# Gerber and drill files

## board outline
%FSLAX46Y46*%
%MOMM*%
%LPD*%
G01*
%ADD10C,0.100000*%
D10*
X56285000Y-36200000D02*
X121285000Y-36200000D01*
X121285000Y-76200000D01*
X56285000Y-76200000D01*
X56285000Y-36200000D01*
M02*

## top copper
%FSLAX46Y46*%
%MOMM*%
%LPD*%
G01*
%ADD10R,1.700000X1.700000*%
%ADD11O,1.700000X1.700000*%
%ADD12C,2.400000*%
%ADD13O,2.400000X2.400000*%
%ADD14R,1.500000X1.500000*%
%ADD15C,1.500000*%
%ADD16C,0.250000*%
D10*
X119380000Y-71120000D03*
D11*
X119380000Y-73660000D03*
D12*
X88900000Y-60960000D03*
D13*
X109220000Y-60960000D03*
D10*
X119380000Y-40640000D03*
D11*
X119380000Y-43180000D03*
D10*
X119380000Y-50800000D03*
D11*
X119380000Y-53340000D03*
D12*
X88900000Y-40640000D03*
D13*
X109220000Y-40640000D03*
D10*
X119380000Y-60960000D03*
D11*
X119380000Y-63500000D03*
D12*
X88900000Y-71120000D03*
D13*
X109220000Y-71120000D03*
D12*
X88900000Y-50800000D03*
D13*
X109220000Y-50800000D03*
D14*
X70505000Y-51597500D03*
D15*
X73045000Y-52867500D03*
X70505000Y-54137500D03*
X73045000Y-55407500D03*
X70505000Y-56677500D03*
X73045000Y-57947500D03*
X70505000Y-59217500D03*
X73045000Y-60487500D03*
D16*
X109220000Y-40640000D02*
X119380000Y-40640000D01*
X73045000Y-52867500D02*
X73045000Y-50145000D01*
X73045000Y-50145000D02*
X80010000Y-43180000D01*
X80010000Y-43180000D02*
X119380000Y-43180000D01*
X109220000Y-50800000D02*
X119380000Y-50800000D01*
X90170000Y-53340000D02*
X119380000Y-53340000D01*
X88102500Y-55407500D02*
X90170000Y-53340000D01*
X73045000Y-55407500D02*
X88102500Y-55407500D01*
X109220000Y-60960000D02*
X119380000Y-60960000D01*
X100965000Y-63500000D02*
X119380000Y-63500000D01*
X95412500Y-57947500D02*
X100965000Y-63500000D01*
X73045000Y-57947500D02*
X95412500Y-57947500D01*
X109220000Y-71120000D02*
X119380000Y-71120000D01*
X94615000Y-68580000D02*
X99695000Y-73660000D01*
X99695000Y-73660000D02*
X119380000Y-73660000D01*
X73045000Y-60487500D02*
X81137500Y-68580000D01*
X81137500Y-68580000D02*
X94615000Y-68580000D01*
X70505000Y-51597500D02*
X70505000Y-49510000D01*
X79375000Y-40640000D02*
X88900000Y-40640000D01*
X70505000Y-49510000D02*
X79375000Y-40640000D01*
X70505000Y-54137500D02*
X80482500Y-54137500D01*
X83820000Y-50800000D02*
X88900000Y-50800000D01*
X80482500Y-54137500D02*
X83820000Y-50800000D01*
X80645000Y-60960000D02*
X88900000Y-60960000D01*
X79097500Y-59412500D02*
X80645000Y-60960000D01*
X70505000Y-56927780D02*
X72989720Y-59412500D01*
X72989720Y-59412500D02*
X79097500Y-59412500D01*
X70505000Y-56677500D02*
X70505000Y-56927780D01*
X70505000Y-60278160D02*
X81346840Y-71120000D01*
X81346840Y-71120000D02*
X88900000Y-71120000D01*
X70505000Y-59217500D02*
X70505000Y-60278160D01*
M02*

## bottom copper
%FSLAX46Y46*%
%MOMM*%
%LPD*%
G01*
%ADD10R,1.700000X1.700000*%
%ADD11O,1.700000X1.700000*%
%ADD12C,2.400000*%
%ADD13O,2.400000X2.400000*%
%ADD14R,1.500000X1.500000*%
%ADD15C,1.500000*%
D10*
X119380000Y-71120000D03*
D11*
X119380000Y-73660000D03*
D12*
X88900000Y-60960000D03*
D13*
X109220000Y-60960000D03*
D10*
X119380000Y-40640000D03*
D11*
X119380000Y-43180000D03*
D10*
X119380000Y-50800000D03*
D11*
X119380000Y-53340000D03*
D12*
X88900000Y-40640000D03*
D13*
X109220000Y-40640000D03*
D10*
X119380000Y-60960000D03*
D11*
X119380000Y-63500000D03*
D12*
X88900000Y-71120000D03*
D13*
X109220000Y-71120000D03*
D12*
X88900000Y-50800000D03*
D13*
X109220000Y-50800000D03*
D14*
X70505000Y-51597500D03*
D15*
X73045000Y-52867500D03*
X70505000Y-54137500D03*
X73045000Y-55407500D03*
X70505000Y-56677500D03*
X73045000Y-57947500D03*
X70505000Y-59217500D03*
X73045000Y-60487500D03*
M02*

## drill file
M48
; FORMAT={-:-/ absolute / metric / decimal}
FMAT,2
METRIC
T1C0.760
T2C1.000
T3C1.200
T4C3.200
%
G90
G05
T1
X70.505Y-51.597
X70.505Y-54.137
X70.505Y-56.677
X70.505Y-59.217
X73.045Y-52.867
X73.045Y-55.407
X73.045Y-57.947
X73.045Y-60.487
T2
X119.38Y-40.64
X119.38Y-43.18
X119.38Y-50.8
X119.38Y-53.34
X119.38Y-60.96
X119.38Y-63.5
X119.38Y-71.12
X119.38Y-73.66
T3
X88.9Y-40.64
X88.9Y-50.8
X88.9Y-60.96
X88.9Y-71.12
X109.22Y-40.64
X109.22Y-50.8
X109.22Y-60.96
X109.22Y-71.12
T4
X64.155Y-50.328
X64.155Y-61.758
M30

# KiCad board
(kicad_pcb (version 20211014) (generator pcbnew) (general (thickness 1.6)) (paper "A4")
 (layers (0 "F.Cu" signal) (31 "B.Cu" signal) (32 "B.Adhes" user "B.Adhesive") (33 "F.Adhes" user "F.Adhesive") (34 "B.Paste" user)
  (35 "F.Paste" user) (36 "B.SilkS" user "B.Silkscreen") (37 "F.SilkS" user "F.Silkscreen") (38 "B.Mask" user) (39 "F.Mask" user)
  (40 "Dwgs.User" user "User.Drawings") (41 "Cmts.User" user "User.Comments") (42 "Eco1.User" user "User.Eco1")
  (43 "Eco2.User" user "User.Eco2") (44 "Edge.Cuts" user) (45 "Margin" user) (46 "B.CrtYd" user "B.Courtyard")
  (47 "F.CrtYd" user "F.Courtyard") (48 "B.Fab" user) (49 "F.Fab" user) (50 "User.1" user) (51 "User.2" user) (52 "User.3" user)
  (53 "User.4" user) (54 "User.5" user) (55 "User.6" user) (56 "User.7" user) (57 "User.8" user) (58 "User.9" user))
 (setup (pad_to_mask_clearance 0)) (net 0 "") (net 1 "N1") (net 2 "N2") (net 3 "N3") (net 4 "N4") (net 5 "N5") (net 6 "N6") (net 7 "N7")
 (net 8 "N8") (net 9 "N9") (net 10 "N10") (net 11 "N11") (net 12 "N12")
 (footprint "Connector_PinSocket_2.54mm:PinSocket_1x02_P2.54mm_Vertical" (layer "F.Cu") (at 119.38 71.12)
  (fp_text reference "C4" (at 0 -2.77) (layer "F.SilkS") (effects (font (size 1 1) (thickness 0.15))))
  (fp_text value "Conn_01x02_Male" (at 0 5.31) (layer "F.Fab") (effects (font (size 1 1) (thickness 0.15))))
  (pad "1" thru_hole rect (at 0 0) (size 1.7 1.7) (drill 1) (layers *.Cu *.Mask) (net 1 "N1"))
  (pad "2" thru_hole oval (at 0 2.54) (size 1.7 1.7) (drill 1) (layers *.Cu *.Mask) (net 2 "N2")))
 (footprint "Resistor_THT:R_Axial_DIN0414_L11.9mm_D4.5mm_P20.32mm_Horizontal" (layer "F.Cu") (at 88.9 60.96)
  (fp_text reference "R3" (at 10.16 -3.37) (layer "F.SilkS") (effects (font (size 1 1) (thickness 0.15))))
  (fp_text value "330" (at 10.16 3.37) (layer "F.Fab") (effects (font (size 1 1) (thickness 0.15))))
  (pad "1" thru_hole circle (at 0 0) (size 2.4 2.4) (drill 1.2) (layers *.Cu *.Mask) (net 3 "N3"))
  (pad "2" thru_hole oval (at 20.32 0) (size 2.4 2.4) (drill 1.2) (layers *.Cu *.Mask) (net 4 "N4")))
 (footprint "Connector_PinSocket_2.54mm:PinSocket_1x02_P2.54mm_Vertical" (layer "F.Cu") (at 119.38 40.64)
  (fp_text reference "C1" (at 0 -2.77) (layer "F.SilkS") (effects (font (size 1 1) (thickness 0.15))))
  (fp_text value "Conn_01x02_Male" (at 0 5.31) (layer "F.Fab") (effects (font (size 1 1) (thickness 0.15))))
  (pad "1" thru_hole rect (at 0 0) (size 1.7 1.7) (drill 1) (layers *.Cu *.Mask) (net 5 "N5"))
  (pad "2" thru_hole oval (at 0 2.54) (size 1.7 1.7) (drill 1) (layers *.Cu *.Mask) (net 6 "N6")))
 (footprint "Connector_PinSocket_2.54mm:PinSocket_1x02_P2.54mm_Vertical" (layer "F.Cu") (at 119.38 50.8)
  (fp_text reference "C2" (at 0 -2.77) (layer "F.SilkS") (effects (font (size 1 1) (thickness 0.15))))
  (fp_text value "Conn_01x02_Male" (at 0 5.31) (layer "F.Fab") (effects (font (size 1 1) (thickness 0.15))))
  (pad "1" thru_hole rect (at 0 0) (size 1.7 1.7) (drill 1) (layers *.Cu *.Mask) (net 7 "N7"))
  (pad "2" thru_hole oval (at 0 2.54) (size 1.7 1.7) (drill 1) (layers *.Cu *.Mask) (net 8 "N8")))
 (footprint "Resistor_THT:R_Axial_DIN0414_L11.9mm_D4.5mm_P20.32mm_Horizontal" (layer "F.Cu") (at 88.9 40.64)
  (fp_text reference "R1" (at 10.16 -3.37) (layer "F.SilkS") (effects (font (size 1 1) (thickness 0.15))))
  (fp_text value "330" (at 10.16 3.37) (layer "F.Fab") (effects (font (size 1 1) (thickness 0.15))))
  (pad "1" thru_hole circle (at 0 0) (size 2.4 2.4) (drill 1.2) (layers *.Cu *.Mask) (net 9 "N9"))
  (pad "2" thru_hole oval (at 20.32 0) (size 2.4 2.4) (drill 1.2) (layers *.Cu *.Mask) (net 5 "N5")))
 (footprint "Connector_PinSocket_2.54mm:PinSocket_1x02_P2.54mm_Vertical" (layer "F.Cu") (at 119.38 60.96)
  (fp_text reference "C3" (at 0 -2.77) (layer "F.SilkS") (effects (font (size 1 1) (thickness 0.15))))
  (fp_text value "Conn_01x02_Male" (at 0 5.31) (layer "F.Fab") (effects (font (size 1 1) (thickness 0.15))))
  (pad "1" thru_hole rect (at 0 0) (size 1.7 1.7) (drill 1) (layers *.Cu *.Mask) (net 4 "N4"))
  (pad "2" thru_hole oval (at 0 2.54) (size 1.7 1.7) (drill 1) (layers *.Cu *.Mask) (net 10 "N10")))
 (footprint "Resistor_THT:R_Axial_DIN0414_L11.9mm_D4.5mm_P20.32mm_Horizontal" (layer "F.Cu") (at 88.9 71.12)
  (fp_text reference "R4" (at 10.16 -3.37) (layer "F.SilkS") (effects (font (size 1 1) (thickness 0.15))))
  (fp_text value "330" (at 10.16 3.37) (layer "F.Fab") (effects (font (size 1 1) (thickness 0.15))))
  (pad "1" thru_hole circle (at 0 0) (size 2.4 2.4) (drill 1.2) (layers *.Cu *.Mask) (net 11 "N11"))
  (pad "2" thru_hole oval (at 20.32 0) (size 2.4 2.4) (drill 1.2) (layers *.Cu *.Mask) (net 1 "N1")))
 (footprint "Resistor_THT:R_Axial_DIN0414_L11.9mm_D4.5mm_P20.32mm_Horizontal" (layer "F.Cu") (at 88.9 50.8)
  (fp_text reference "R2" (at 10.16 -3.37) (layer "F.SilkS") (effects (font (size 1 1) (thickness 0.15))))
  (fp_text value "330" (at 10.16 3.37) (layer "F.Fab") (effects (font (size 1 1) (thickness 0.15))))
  (pad "1" thru_hole circle (at 0 0) (size 2.4 2.4) (drill 1.2) (layers *.Cu *.Mask) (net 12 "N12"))
  (pad "2" thru_hole oval (at 20.32 0) (size 2.4 2.4) (drill 1.2) (layers *.Cu *.Mask) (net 7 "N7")))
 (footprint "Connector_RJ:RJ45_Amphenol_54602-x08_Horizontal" (layer "F.Cu") (at 70.505 51.5975 -90)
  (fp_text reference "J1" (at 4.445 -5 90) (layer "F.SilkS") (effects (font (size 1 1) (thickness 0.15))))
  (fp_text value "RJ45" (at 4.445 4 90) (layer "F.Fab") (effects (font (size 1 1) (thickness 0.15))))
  (pad "" np_thru_hole circle (at 10.16 6.35 270) (size 3.2 3.2) (drill 3.2) (layers *.Cu *.Mask))
  (pad "" np_thru_hole circle (at -1.27 6.35 270) (size 3.2 3.2) (drill 3.2) (layers *.Cu *.Mask))
  (pad "1" thru_hole rect (at 0 0 270) (size 1.5 1.5) (drill 0.76) (layers *.Cu *.Mask) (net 9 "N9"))
  (pad "2" thru_hole circle (at 1.27 -2.54 270) (size 1.5 1.5) (drill 0.76) (layers *.Cu *.Mask) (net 6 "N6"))
  (pad "3" thru_hole circle (at 2.54 0 270) (size 1.5 1.5) (drill 0.76) (layers *.Cu *.Mask) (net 12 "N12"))
  (pad "4" thru_hole circle (at 3.81 -2.54 270) (size 1.5 1.5) (drill 0.76) (layers *.Cu *.Mask) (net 8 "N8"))
  (pad "5" thru_hole circle (at 5.08 0 270) (size 1.5 1.5) (drill 0.76) (layers *.Cu *.Mask) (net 3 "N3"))
  (pad "6" thru_hole circle (at 6.35 -2.54 270) (size 1.5 1.5) (drill 0.76) (layers *.Cu *.Mask) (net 10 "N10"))
  (pad "7" thru_hole circle (at 7.62 0 270) (size 1.5 1.5) (drill 0.76) (layers *.Cu *.Mask) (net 11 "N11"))
  (pad "8" thru_hole circle (at 8.89 -2.54 270) (size 1.5 1.5) (drill 0.76) (layers *.Cu *.Mask) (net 2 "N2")))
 (gr_rect (start 56.285 36.2) (end 121.285 76.2) (layer "Edge.Cuts") (width 0.1) (fill none))
 (segment (start 109.22 40.64) (end 119.38 40.64) (width 0.25) (layer "F.Cu") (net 5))
 (segment (start 73.045 52.8675) (end 73.045 50.145) (width 0.25) (layer "F.Cu") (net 6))
 (segment (start 73.045 50.145) (end 80.01 43.18) (width 0.25) (layer "F.Cu") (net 6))
 (segment (start 80.01 43.18) (end 119.38 43.18) (width 0.25) (layer "F.Cu") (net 6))
 (segment (start 109.22 50.8) (end 119.38 50.8) (width 0.25) (layer "F.Cu") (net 7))
 (segment (start 90.17 53.34) (end 119.38 53.34) (width 0.25) (layer "F.Cu") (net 8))
 (segment (start 88.1025 55.4075) (end 90.17 53.34) (width 0.25) (layer "F.Cu") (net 8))
 (segment (start 73.045 55.4075) (end 88.1025 55.4075) (width 0.25) (layer "F.Cu") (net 8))
 (segment (start 109.22 60.96) (end 119.38 60.96) (width 0.25) (layer "F.Cu") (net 4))
 (segment (start 100.965 63.5) (end 119.38 63.5) (width 0.25) (layer "F.Cu") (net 10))
 (segment (start 95.4125 57.9475) (end 100.965 63.5) (width 0.25) (layer "F.Cu") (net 10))
 (segment (start 73.045 57.9475) (end 95.4125 57.9475) (width 0.25) (layer "F.Cu") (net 10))
 (segment (start 109.22 71.12) (end 119.38 71.12) (width 0.25) (layer "F.Cu") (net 1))
 (segment (start 94.615 68.58) (end 99.695 73.66) (width 0.25) (layer "F.Cu") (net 2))
 (segment (start 99.695 73.66) (end 119.38 73.66) (width 0.25) (layer "F.Cu") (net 2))
 (segment (start 73.045 60.4875) (end 81.1375 68.58) (width 0.25) (layer "F.Cu") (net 2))
 (segment (start 81.1375 68.58) (end 94.615 68.58) (width 0.25) (layer "F.Cu") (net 2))
 (segment (start 70.505 51.5975) (end 70.505 49.51) (width 0.25) (layer "F.Cu") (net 9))
 (segment (start 79.375 40.64) (end 88.9 40.64) (width 0.25) (layer "F.Cu") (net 9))
 (segment (start 70.505 49.51) (end 79.375 40.64) (width 0.25) (layer "F.Cu") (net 9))
 (segment (start 70.505 54.1375) (end 80.4825 54.1375) (width 0.25) (layer "F.Cu") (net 12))
 (segment (start 83.82 50.8) (end 88.9 50.8) (width 0.25) (layer "F.Cu") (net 12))
 (segment (start 80.4825 54.1375) (end 83.82 50.8) (width 0.25) (layer "F.Cu") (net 12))
 (segment (start 80.645 60.96) (end 88.9 60.96) (width 0.25) (layer "F.Cu") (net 3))
 (segment (start 79.0975 59.4125) (end 80.645 60.96) (width 0.25) (layer "F.Cu") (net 3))
 (segment (start 70.505 56.92778) (end 72.98972 59.4125) (width 0.25) (layer "F.Cu") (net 3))
 (segment (start 72.98972 59.4125) (end 79.0975 59.4125) (width 0.25) (layer "F.Cu") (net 3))
 (segment (start 70.505 56.6775) (end 70.505 56.92778) (width 0.25) (layer "F.Cu") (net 3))
 (segment (start 70.505 60.27816) (end 81.34684 71.12) (width 0.25) (layer "F.Cu") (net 11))
 (segment (start 81.34684 71.12) (end 88.9 71.12) (width 0.25) (layer "F.Cu") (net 11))
 (segment (start 70.505 59.2175) (end 70.505 60.27816) (width 0.25) (layer "F.Cu") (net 11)))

